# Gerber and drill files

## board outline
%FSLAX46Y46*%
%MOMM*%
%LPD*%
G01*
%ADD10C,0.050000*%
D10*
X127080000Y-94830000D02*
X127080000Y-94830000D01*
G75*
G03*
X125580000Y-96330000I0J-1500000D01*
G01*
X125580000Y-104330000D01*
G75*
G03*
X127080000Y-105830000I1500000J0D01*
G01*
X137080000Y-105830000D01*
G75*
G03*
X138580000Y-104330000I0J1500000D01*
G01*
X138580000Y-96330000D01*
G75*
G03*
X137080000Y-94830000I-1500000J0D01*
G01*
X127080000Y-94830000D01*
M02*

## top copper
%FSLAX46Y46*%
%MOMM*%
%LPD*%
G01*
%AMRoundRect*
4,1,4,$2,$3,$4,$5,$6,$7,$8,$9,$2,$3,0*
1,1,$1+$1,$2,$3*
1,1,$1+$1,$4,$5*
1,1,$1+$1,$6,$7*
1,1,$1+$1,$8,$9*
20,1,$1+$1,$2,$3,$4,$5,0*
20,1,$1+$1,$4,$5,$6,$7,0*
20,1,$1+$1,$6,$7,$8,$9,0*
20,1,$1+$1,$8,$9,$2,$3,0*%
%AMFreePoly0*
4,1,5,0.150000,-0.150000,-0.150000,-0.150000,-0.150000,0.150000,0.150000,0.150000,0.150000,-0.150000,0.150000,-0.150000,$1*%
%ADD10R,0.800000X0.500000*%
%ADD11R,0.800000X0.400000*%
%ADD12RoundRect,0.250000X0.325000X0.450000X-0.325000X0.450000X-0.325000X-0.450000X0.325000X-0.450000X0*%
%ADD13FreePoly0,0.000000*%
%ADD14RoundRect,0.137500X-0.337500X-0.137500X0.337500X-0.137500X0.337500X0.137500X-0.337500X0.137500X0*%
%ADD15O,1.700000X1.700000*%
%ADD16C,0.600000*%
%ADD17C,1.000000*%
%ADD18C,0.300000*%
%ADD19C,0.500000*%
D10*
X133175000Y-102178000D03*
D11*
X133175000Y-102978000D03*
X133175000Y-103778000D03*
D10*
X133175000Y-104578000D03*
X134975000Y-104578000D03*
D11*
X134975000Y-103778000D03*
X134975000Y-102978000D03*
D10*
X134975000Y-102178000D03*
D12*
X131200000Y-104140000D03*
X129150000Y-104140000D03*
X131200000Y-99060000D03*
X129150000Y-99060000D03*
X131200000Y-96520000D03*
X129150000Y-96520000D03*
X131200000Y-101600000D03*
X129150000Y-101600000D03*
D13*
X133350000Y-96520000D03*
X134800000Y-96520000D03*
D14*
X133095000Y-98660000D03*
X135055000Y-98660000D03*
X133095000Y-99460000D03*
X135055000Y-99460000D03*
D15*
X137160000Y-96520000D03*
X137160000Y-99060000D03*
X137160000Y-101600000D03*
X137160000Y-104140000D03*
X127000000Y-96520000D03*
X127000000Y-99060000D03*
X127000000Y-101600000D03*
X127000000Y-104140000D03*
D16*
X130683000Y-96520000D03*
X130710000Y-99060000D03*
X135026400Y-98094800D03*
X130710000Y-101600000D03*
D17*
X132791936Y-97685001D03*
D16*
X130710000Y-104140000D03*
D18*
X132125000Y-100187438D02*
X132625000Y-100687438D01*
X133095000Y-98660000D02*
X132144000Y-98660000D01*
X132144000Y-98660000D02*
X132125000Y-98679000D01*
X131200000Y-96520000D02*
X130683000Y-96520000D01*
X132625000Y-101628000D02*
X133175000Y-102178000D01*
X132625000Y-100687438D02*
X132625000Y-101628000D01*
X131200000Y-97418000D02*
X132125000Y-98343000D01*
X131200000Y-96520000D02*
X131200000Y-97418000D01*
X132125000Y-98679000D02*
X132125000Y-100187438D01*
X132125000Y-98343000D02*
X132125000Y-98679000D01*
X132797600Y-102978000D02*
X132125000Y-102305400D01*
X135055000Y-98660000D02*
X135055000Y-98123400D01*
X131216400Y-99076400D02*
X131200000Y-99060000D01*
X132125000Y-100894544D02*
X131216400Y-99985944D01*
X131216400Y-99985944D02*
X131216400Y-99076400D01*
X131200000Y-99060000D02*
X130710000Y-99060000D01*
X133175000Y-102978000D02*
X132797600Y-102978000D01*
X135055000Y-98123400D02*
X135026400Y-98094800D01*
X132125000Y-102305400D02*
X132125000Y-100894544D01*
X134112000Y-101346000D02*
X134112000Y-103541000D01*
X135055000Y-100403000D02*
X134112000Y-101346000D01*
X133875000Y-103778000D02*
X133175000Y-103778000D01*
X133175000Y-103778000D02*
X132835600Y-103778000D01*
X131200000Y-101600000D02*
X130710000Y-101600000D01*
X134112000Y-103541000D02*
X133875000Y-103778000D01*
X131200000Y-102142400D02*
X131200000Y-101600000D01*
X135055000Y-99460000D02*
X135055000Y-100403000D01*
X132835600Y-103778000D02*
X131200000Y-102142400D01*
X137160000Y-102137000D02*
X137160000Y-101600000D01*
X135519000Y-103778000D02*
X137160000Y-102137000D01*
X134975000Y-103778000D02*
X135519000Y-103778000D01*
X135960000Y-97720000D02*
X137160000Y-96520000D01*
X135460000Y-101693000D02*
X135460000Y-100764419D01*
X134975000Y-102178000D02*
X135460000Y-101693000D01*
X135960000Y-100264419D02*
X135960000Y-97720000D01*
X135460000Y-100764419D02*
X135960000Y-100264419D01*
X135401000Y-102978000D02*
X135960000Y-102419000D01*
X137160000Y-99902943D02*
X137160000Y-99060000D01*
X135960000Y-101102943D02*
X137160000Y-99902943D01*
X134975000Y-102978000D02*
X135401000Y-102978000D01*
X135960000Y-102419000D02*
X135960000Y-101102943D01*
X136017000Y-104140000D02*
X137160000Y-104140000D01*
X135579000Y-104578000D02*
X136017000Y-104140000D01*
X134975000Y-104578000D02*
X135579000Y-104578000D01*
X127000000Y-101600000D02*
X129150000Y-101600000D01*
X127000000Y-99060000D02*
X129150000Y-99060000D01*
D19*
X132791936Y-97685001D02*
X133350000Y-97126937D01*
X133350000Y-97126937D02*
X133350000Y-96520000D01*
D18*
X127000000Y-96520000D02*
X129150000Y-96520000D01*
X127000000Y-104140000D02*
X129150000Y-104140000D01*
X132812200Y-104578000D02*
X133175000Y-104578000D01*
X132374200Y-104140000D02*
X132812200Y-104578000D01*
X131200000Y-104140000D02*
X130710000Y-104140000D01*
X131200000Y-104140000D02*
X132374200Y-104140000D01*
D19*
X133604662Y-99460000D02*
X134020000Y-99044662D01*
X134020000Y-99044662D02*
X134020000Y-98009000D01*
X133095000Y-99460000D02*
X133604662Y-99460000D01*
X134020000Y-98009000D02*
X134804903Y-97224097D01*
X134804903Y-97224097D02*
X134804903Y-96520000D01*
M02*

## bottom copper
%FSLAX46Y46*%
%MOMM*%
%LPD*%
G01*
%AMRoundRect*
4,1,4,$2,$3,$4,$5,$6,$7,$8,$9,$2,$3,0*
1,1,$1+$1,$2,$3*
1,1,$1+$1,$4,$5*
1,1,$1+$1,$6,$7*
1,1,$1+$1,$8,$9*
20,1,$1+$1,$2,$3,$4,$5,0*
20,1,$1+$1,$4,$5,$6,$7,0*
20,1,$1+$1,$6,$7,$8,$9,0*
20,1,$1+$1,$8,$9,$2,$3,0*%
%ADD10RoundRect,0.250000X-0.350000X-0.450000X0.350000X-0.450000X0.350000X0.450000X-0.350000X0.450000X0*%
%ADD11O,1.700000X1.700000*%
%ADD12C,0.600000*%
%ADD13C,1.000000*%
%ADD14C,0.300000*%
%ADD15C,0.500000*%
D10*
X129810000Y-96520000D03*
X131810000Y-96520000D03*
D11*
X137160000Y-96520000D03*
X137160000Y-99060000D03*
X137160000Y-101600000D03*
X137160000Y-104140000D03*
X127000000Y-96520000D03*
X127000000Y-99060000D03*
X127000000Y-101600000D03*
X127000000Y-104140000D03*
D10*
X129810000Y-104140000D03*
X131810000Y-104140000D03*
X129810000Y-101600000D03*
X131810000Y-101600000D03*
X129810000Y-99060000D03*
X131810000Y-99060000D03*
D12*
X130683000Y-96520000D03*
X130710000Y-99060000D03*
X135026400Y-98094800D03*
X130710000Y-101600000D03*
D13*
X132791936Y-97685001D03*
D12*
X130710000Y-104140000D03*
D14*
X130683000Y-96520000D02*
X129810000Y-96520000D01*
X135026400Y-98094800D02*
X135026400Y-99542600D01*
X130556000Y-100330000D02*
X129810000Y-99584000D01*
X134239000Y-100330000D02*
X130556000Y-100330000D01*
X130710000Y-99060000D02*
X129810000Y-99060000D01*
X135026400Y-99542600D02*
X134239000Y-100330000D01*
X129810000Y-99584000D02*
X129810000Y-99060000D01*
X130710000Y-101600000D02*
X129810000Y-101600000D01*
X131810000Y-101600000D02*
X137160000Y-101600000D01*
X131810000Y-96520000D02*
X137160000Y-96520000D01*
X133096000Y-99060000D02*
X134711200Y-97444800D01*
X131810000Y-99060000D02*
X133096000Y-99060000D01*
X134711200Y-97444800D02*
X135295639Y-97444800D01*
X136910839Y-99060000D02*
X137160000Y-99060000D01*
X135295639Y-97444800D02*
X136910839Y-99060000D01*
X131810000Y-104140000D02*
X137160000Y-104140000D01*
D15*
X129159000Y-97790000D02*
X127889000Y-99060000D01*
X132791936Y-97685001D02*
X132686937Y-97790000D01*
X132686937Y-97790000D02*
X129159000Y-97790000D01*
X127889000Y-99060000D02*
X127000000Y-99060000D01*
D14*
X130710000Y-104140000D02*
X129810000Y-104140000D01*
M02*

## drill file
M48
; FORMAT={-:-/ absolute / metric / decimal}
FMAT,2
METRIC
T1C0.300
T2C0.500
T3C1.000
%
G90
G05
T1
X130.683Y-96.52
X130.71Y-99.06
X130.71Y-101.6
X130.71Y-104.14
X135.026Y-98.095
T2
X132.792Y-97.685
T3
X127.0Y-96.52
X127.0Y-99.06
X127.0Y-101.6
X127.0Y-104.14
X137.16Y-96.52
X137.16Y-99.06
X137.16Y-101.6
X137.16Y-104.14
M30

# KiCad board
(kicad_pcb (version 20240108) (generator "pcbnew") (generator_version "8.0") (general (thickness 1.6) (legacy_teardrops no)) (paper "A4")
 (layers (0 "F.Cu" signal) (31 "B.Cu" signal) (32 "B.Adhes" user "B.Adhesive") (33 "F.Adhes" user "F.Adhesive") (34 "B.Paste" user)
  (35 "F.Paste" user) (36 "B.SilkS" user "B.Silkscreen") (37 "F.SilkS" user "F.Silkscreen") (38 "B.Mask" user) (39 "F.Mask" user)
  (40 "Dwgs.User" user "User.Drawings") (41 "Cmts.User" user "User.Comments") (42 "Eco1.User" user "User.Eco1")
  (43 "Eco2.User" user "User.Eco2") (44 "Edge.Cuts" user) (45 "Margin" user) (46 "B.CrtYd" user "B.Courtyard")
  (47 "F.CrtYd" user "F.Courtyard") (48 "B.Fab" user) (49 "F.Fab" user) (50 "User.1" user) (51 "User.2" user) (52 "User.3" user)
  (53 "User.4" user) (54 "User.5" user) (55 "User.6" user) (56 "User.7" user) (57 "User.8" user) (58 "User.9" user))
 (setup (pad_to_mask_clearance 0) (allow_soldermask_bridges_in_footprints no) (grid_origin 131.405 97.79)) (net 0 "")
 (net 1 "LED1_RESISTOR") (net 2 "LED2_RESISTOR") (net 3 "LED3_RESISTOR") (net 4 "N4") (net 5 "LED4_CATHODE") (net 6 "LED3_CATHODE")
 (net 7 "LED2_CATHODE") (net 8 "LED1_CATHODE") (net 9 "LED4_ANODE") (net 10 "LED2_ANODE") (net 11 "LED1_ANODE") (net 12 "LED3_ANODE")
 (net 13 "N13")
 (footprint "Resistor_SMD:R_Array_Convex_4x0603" (layer "F.Cu") (at 134.075 103.378)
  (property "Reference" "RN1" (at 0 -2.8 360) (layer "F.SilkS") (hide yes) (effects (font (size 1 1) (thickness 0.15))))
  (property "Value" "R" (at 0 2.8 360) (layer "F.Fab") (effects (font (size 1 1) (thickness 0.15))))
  (pad "1" smd rect (at -0.9 -1.2) (size 0.8 0.5) (layers "F.Cu" "F.Paste" "F.Mask") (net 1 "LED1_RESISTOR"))
  (pad "2" smd rect (at -0.9 -0.4) (size 0.8 0.4) (layers "F.Cu" "F.Paste" "F.Mask") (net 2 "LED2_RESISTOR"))
  (pad "3" smd rect (at -0.9 0.4) (size 0.8 0.4) (layers "F.Cu" "F.Paste" "F.Mask") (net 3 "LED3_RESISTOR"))
  (pad "4" smd rect (at -0.9 1.2) (size 0.8 0.5) (layers "F.Cu" "F.Paste" "F.Mask") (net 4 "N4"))
  (pad "5" smd rect (at 0.9 1.2) (size 0.8 0.5) (layers "F.Cu" "F.Paste" "F.Mask") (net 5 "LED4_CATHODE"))
  (pad "6" smd rect (at 0.9 0.4) (size 0.8 0.4) (layers "F.Cu" "F.Paste" "F.Mask") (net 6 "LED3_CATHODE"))
  (pad "7" smd rect (at 0.9 -0.4) (size 0.8 0.4) (layers "F.Cu" "F.Paste" "F.Mask") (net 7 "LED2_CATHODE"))
  (pad "8" smd rect (at 0.9 -1.2) (size 0.8 0.5) (layers "F.Cu" "F.Paste" "F.Mask") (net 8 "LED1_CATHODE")))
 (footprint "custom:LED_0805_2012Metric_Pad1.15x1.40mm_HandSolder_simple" (layer "F.Cu") (at 130.175 104.14 180)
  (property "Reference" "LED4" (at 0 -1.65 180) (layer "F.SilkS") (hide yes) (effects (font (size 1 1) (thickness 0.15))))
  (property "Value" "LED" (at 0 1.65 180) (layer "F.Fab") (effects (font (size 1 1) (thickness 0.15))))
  (pad "1" smd roundrect (at -1.025 0 180) (size 1.15 1.4) (layers "F.Cu" "F.Paste" "F.Mask") (roundrect_rratio 0.217391) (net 4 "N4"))
  (pad "2" smd roundrect (at 1.025 0 180) (size 1.15 1.4) (layers "F.Cu" "F.Paste" "F.Mask") (roundrect_rratio 0.217391)
   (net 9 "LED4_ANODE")))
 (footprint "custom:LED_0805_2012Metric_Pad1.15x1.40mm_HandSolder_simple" (layer "F.Cu") (at 130.175 99.06 180)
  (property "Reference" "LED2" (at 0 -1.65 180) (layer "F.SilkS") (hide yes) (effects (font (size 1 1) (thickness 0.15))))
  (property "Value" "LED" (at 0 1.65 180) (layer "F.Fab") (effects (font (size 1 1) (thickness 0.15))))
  (pad "1" smd roundrect (at -1.025 0 180) (size 1.15 1.4) (layers "F.Cu" "F.Paste" "F.Mask") (roundrect_rratio 0.217391)
   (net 2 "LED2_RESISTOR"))
  (pad "2" smd roundrect (at 1.025 0 180) (size 1.15 1.4) (layers "F.Cu" "F.Paste" "F.Mask") (roundrect_rratio 0.217391)
   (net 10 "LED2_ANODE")))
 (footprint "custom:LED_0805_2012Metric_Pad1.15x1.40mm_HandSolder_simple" (layer "F.Cu") (at 130.175 96.52 180)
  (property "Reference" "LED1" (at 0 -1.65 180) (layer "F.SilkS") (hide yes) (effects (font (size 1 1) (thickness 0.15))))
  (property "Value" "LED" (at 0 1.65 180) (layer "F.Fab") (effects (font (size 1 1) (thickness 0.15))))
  (pad "1" smd roundrect (at -1.025 0 180) (size 1.15 1.4) (layers "F.Cu" "F.Paste" "F.Mask") (roundrect_rratio 0.217391)
   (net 1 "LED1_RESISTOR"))
  (pad "2" smd roundrect (at 1.025 0 180) (size 1.15 1.4) (layers "F.Cu" "F.Paste" "F.Mask") (roundrect_rratio 0.217391)
   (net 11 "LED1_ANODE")))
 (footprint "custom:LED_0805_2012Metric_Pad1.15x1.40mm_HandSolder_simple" (layer "F.Cu") (at 130.175 101.6 180)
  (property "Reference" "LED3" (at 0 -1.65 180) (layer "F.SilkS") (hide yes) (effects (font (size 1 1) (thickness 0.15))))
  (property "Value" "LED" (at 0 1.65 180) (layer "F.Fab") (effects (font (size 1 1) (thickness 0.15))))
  (pad "1" smd roundrect (at -1.025 0 180) (size 1.15 1.4) (layers "F.Cu" "F.Paste" "F.Mask") (roundrect_rratio 0.217391)
   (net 3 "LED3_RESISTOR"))
  (pad "2" smd roundrect (at 1.025 0 180) (size 1.15 1.4) (layers "F.Cu" "F.Paste" "F.Mask") (roundrect_rratio 0.217391)
   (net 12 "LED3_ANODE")))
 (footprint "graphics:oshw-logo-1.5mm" (layer "F.Cu") (at 134.874 100.711)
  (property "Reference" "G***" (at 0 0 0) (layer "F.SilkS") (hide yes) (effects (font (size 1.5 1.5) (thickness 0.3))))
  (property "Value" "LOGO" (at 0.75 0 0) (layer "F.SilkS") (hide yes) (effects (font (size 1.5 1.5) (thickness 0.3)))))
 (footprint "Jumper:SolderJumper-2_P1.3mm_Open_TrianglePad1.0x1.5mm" (layer "F.Cu") (at 134.075 96.52)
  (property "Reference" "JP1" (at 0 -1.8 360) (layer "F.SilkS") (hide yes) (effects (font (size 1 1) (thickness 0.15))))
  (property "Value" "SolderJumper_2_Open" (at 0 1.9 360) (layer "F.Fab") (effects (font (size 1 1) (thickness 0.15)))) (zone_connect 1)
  (pad "1" smd custom (at -0.725 0) (size 0.3 0.3) (layers "F.Cu" "F.Mask") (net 10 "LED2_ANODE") (zone_connect 2) (thermal_bridge_angle 45)
   (options (clearance outline) (anchor rect)) (primitives))
  (pad "2" smd custom (at 0.725 0) (size 0.3 0.3) (layers "F.Cu" "F.Mask") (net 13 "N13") (zone_connect 2) (thermal_bridge_angle 45)
   (options (clearance outline) (anchor rect)) (primitives)))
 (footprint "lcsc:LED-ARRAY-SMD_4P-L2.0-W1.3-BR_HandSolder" (layer "F.Cu") (at 134.075 99.06 180)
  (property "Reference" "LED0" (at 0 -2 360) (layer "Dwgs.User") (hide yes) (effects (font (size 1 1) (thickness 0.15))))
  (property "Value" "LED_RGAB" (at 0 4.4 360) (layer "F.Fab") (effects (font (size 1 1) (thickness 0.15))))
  (pad "1" smd roundrect (at 0.98 0.4) (size 0.95 0.55) (layers "F.Cu" "F.Paste" "F.Mask") (roundrect_rratio 0.25) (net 1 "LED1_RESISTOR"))
  (pad "2" smd roundrect (at -0.98 0.4) (size 0.95 0.55) (layers "F.Cu" "F.Paste" "F.Mask") (roundrect_rratio 0.25) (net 2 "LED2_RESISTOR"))
  (pad "3" smd roundrect (at 0.98 -0.4) (size 0.95 0.55) (layers "F.Cu" "F.Paste" "F.Mask") (roundrect_rratio 0.25) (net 13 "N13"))
  (pad "4" smd roundrect (at -0.98 -0.4) (size 0.95 0.55) (layers "F.Cu" "F.Paste" "F.Mask") (roundrect_rratio 0.25) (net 3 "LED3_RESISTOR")))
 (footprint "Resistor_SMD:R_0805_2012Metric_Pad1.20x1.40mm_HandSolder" (layer "B.Cu") (at 130.81 96.52)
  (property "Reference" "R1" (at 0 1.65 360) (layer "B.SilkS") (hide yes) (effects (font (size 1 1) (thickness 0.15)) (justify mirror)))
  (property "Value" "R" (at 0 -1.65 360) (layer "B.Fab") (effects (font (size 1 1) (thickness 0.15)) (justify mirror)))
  (pad "1" smd roundrect (at -1 0) (size 1.2 1.4) (layers "B.Cu" "B.Paste" "B.Mask") (roundrect_rratio 0.208333) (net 1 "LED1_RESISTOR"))
  (pad "2" smd roundrect (at 1 0) (size 1.2 1.4) (layers "B.Cu" "B.Paste" "B.Mask") (roundrect_rratio 0.208333) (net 8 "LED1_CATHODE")))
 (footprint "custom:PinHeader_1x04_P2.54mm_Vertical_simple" (layer "B.Cu") (at 137.16 96.52 180)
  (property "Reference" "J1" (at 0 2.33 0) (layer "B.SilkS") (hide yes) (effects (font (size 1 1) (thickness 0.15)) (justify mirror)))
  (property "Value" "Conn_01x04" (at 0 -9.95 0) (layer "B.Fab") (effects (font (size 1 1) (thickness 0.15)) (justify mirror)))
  (pad "1" thru_hole oval (at 0 0 180) (size 1.7 1.7) (drill 1) (layers "*.Cu" "*.Mask") (remove_unused_layers no) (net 8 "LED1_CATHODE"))
  (pad "2" thru_hole oval (at 0 -2.54 180) (size 1.7 1.7) (drill 1) (layers "*.Cu" "*.Mask") (remove_unused_layers no)
   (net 7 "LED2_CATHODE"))
  (pad "3" thru_hole oval (at 0 -5.08 180) (size 1.7 1.7) (drill 1) (layers "*.Cu" "*.Mask") (remove_unused_layers no)
   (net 6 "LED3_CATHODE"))
  (pad "4" thru_hole oval (at 0 -7.62 180) (size 1.7 1.7) (drill 1) (layers "*.Cu" "*.Mask") (remove_unused_layers no)
   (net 5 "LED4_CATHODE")))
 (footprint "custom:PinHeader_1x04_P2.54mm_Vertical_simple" (layer "B.Cu") (at 127 96.52 180)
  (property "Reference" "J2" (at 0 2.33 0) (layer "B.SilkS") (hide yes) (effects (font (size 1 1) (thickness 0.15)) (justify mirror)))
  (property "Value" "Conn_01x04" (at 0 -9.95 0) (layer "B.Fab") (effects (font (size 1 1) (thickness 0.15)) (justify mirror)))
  (pad "1" thru_hole oval (at 0 0 180) (size 1.7 1.7) (drill 1) (layers "*.Cu" "*.Mask") (remove_unused_layers no) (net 11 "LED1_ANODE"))
  (pad "2" thru_hole oval (at 0 -2.54 180) (size 1.7 1.7) (drill 1) (layers "*.Cu" "*.Mask") (remove_unused_layers no) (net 10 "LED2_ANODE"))
  (pad "3" thru_hole oval (at 0 -5.08 180) (size 1.7 1.7) (drill 1) (layers "*.Cu" "*.Mask") (remove_unused_layers no) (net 12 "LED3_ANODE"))
  (pad "4" thru_hole oval (at 0 -7.62 180) (size 1.7 1.7) (drill 1) (layers "*.Cu" "*.Mask") (remove_unused_layers no) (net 9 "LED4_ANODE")))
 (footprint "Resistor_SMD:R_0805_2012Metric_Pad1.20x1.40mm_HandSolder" (layer "B.Cu") (at 130.81 104.14)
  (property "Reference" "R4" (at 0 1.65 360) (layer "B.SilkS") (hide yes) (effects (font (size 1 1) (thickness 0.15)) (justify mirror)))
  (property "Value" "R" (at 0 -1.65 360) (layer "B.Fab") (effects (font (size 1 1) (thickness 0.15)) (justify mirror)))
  (pad "1" smd roundrect (at -1 0) (size 1.2 1.4) (layers "B.Cu" "B.Paste" "B.Mask") (roundrect_rratio 0.208333) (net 4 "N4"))
  (pad "2" smd roundrect (at 1 0) (size 1.2 1.4) (layers "B.Cu" "B.Paste" "B.Mask") (roundrect_rratio 0.208333) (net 5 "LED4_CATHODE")))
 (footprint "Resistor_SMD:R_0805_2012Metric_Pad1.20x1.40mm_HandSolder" (layer "B.Cu") (at 130.81 101.6)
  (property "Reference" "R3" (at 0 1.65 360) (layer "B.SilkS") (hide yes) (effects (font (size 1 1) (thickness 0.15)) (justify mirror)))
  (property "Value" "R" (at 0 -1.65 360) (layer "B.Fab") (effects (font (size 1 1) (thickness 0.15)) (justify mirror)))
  (pad "1" smd roundrect (at -1 0) (size 1.2 1.4) (layers "B.Cu" "B.Paste" "B.Mask") (roundrect_rratio 0.208333) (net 3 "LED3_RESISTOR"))
  (pad "2" smd roundrect (at 1 0) (size 1.2 1.4) (layers "B.Cu" "B.Paste" "B.Mask") (roundrect_rratio 0.208333) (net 6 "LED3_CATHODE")))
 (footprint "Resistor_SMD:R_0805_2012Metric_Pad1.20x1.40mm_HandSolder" (layer "B.Cu") (at 130.81 99.06)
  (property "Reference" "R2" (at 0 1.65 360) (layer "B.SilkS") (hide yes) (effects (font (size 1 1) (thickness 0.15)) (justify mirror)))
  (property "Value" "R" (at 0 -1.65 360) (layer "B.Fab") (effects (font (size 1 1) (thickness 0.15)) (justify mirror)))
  (pad "1" smd roundrect (at -1 0) (size 1.2 1.4) (layers "B.Cu" "B.Paste" "B.Mask") (roundrect_rratio 0.208333) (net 2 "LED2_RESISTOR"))
  (pad "2" smd roundrect (at 1 0) (size 1.2 1.4) (layers "B.Cu" "B.Paste" "B.Mask") (roundrect_rratio 0.208333) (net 7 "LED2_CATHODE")))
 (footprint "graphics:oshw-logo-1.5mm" (layer "B.Cu") (at 133.55 98.75 90)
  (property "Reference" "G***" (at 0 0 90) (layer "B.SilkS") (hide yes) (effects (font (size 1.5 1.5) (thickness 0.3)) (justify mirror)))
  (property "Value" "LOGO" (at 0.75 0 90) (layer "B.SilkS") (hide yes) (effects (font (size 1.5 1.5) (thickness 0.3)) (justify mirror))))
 (gr_poly
  (pts
   (arc (start 127.08 94.83) (mid 126.01934 95.26934) (end 125.58 96.33))
   (arc (start 125.58 104.33) (mid 126.01934 105.39066) (end 127.08 105.83))
   (arc (start 137.08 105.83) (mid 138.14066 105.39066) (end 138.58 104.33))
   (arc (start 138.58 96.33) (mid 138.14066 95.26934) (end 137.08 94.83)))
  (stroke (width 0.05) (type solid)) (fill none) (layer "Edge.Cuts"))
 (segment (start 132.125 100.187438) (end 132.625 100.687438) (width 0.3) (layer "F.Cu") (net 1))
 (segment (start 133.095 98.66) (end 132.144 98.66) (width 0.3) (layer "F.Cu") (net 1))
 (segment (start 132.144 98.66) (end 132.125 98.679) (width 0.3) (layer "F.Cu") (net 1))
 (segment (start 131.2 96.52) (end 130.683 96.52) (width 0.3) (layer "F.Cu") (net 1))
 (segment (start 132.625 101.628) (end 133.175 102.178) (width 0.3) (layer "F.Cu") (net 1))
 (segment (start 132.625 100.687438) (end 132.625 101.628) (width 0.3) (layer "F.Cu") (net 1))
 (segment (start 131.2 97.418) (end 132.125 98.343) (width 0.3) (layer "F.Cu") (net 1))
 (segment (start 131.2 96.52) (end 131.2 97.418) (width 0.3) (layer "F.Cu") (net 1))
 (segment (start 132.125 98.679) (end 132.125 100.187438) (width 0.3) (layer "F.Cu") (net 1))
 (segment (start 132.125 98.343) (end 132.125 98.679) (width 0.3) (layer "F.Cu") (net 1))
 (via (at 130.683 96.52) (size 0.6) (drill 0.3) (layers "F.Cu" "B.Cu") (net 1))
 (segment (start 130.683 96.52) (end 129.81 96.52) (width 0.3) (layer "B.Cu") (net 1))
 (segment (start 132.7976 102.978) (end 132.125 102.3054) (width 0.3) (layer "F.Cu") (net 2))
 (segment (start 135.055 98.66) (end 135.055 98.1234) (width 0.3) (layer "F.Cu") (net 2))
 (segment (start 131.2164 99.0764) (end 131.2 99.06) (width 0.3) (layer "F.Cu") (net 2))
 (segment (start 132.125 100.894544) (end 131.2164 99.985944) (width 0.3) (layer "F.Cu") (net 2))
 (segment (start 131.2164 99.985944) (end 131.2164 99.0764) (width 0.3) (layer "F.Cu") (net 2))
 (segment (start 131.2 99.06) (end 130.71 99.06) (width 0.3) (layer "F.Cu") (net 2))
 (segment (start 133.175 102.978) (end 132.7976 102.978) (width 0.3) (layer "F.Cu") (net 2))
 (segment (start 135.055 98.1234) (end 135.0264 98.0948) (width 0.3) (layer "F.Cu") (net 2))
 (segment (start 132.125 102.3054) (end 132.125 100.894544) (width 0.3) (layer "F.Cu") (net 2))
 (via (at 130.71 99.06) (size 0.6) (drill 0.3) (layers "F.Cu" "B.Cu") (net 2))
 (via (at 135.0264 98.0948) (size 0.6) (drill 0.3) (layers "F.Cu" "B.Cu") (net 2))
 (segment (start 135.0264 98.0948) (end 135.0264 99.5426) (width 0.3) (layer "B.Cu") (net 2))
 (segment (start 130.556 100.33) (end 129.81 99.584) (width 0.3) (layer "B.Cu") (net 2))
 (segment (start 134.239 100.33) (end 130.556 100.33) (width 0.3) (layer "B.Cu") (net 2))
 (segment (start 130.71 99.06) (end 129.81 99.06) (width 0.3) (layer "B.Cu") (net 2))
 (segment (start 135.0264 99.5426) (end 134.239 100.33) (width 0.3) (layer "B.Cu") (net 2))
 (segment (start 129.81 99.584) (end 129.81 99.06) (width 0.3) (layer "B.Cu") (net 2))
 (segment (start 134.112 101.346) (end 134.112 103.541) (width 0.3) (layer "F.Cu") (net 3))
 (segment (start 135.055 100.403) (end 134.112 101.346) (width 0.3) (layer "F.Cu") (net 3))
 (segment (start 133.875 103.778) (end 133.175 103.778) (width 0.3) (layer "F.Cu") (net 3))
 (segment (start 133.175 103.778) (end 132.8356 103.778) (width 0.3) (layer "F.Cu") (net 3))
 (segment (start 131.2 101.6) (end 130.71 101.6) (width 0.3) (layer "F.Cu") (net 3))
 (segment (start 134.112 103.541) (end 133.875 103.778) (width 0.3) (layer "F.Cu") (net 3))
 (segment (start 131.2 102.1424) (end 131.2 101.6) (width 0.3) (layer "F.Cu") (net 3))
 (segment (start 135.055 99.46) (end 135.055 100.403) (width 0.3) (layer "F.Cu") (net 3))
 (segment (start 132.8356 103.778) (end 131.2 102.1424) (width 0.3) (layer "F.Cu") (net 3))
 (via (at 130.71 101.6) (size 0.6) (drill 0.3) (layers "F.Cu" "B.Cu") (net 3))
 (segment (start 130.71 101.6) (end 129.81 101.6) (width 0.3) (layer "B.Cu") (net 3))
 (segment (start 137.16 102.137) (end 137.16 101.6) (width 0.3) (layer "F.Cu") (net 6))
 (segment (start 135.519 103.778) (end 137.16 102.137) (width 0.3) (layer "F.Cu") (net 6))
 (segment (start 134.975 103.778) (end 135.519 103.778) (width 0.3) (layer "F.Cu") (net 6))
 (segment (start 131.81 101.6) (end 137.16 101.6) (width 0.3) (layer "B.Cu") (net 6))
 (segment (start 135.96 97.72) (end 137.16 96.52) (width 0.3) (layer "F.Cu") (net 8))
 (segment (start 135.46 101.693) (end 135.46 100.764419) (width 0.3) (layer "F.Cu") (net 8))
 (segment (start 134.975 102.178) (end 135.46 101.693) (width 0.3) (layer "F.Cu") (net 8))
 (segment (start 135.96 100.264419) (end 135.96 97.72) (width 0.3) (layer "F.Cu") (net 8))
 (segment (start 135.46 100.764419) (end 135.96 100.264419) (width 0.3) (layer "F.Cu") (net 8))
 (segment (start 131.81 96.52) (end 137.16 96.52) (width 0.3) (layer "B.Cu") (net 8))
 (segment (start 135.401 102.978) (end 135.96 102.419) (width 0.3) (layer "F.Cu") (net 7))
 (segment (start 137.16 99.902943) (end 137.16 99.06) (width 0.3) (layer "F.Cu") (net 7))
 (segment (start 135.96 101.102943) (end 137.16 99.902943) (width 0.3) (layer "F.Cu") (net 7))
 (segment (start 134.975 102.978) (end 135.401 102.978) (width 0.3) (layer "F.Cu") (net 7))
 (segment (start 135.96 102.419) (end 135.96 101.102943) (width 0.3) (layer "F.Cu") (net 7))
 (segment (start 133.096 99.06) (end 134.7112 97.4448) (width 0.3) (layer "B.Cu") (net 7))
 (segment (start 131.81 99.06) (end 133.096 99.06) (width 0.3) (layer "B.Cu") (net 7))
 (segment (start 134.7112 97.4448) (end 135.295639 97.4448) (width 0.3) (layer "B.Cu") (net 7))
 (segment (start 136.910839 99.06) (end 137.16 99.06) (width 0.3) (layer "B.Cu") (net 7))
 (segment (start 135.295639 97.4448) (end 136.910839 99.06) (width 0.3) (layer "B.Cu") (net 7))
 (segment (start 136.017 104.14) (end 137.16 104.14) (width 0.3) (layer "F.Cu") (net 5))
 (segment (start 135.579 104.578) (end 136.017 104.14) (width 0.3) (layer "F.Cu") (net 5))
 (segment (start 134.975 104.578) (end 135.579 104.578) (width 0.3) (layer "F.Cu") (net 5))
 (segment (start 131.81 104.14) (end 137.16 104.14) (width 0.3) (layer "B.Cu") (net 5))
 (segment (start 127 101.6) (end 129.15 101.6) (width 0.3) (layer "F.Cu") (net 12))
 (segment (start 127 99.06) (end 129.15 99.06) (width 0.3) (layer "F.Cu") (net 10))
 (segment (start 132.791936 97.685001) (end 133.35 97.126937) (width 0.5) (layer "F.Cu") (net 10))
 (segment (start 133.35 97.126937) (end 133.35 96.52) (width 0.5) (layer "F.Cu") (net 10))
 (via (at 132.791936 97.685001) (size 1) (drill 0.5) (layers "F.Cu" "B.Cu") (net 10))
 (segment (start 129.159 97.79) (end 127.889 99.06) (width 0.5) (layer "B.Cu") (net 10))
 (segment (start 132.791936 97.685001) (end 132.686937 97.79) (width 0.5) (layer "B.Cu") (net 10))
 (segment (start 132.686937 97.79) (end 129.159 97.79) (width 0.5) (layer "B.Cu") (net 10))
 (segment (start 127.889 99.06) (end 127 99.06) (width 0.5) (layer "B.Cu") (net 10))
 (segment (start 127 96.52) (end 129.15 96.52) (width 0.3) (layer "F.Cu") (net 11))
 (segment (start 127 104.14) (end 129.15 104.14) (width 0.3) (layer "F.Cu") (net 9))
 (segment (start 132.8122 104.578) (end 133.175 104.578) (width 0.3) (layer "F.Cu") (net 4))
 (segment (start 132.3742 104.14) (end 132.8122 104.578) (width 0.3) (layer "F.Cu") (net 4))
 (segment (start 131.2 104.14) (end 130.71 104.14) (width 0.3) (layer "F.Cu") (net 4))
 (segment (start 131.2 104.14) (end 132.3742 104.14) (width 0.3) (layer "F.Cu") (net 4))
 (via (at 130.71 104.14) (size 0.6) (drill 0.3) (layers "F.Cu" "B.Cu") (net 4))
 (segment (start 130.71 104.14) (end 129.81 104.14) (width 0.3) (layer "B.Cu") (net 4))
 (segment (start 133.604662 99.46) (end 134.02 99.044662) (width 0.5) (layer "F.Cu") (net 13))
 (segment (start 134.02 99.044662) (end 134.02 98.009) (width 0.5) (layer "F.Cu") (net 13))
 (segment (start 133.095 99.46) (end 133.604662 99.46) (width 0.5) (layer "F.Cu") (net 13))
 (segment (start 134.02 98.009) (end 134.804903 97.224097) (width 0.5) (layer "F.Cu") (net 13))
 (segment (start 134.804903 97.224097) (end 134.804903 96.52) (width 0.5) (layer "F.Cu") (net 13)))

